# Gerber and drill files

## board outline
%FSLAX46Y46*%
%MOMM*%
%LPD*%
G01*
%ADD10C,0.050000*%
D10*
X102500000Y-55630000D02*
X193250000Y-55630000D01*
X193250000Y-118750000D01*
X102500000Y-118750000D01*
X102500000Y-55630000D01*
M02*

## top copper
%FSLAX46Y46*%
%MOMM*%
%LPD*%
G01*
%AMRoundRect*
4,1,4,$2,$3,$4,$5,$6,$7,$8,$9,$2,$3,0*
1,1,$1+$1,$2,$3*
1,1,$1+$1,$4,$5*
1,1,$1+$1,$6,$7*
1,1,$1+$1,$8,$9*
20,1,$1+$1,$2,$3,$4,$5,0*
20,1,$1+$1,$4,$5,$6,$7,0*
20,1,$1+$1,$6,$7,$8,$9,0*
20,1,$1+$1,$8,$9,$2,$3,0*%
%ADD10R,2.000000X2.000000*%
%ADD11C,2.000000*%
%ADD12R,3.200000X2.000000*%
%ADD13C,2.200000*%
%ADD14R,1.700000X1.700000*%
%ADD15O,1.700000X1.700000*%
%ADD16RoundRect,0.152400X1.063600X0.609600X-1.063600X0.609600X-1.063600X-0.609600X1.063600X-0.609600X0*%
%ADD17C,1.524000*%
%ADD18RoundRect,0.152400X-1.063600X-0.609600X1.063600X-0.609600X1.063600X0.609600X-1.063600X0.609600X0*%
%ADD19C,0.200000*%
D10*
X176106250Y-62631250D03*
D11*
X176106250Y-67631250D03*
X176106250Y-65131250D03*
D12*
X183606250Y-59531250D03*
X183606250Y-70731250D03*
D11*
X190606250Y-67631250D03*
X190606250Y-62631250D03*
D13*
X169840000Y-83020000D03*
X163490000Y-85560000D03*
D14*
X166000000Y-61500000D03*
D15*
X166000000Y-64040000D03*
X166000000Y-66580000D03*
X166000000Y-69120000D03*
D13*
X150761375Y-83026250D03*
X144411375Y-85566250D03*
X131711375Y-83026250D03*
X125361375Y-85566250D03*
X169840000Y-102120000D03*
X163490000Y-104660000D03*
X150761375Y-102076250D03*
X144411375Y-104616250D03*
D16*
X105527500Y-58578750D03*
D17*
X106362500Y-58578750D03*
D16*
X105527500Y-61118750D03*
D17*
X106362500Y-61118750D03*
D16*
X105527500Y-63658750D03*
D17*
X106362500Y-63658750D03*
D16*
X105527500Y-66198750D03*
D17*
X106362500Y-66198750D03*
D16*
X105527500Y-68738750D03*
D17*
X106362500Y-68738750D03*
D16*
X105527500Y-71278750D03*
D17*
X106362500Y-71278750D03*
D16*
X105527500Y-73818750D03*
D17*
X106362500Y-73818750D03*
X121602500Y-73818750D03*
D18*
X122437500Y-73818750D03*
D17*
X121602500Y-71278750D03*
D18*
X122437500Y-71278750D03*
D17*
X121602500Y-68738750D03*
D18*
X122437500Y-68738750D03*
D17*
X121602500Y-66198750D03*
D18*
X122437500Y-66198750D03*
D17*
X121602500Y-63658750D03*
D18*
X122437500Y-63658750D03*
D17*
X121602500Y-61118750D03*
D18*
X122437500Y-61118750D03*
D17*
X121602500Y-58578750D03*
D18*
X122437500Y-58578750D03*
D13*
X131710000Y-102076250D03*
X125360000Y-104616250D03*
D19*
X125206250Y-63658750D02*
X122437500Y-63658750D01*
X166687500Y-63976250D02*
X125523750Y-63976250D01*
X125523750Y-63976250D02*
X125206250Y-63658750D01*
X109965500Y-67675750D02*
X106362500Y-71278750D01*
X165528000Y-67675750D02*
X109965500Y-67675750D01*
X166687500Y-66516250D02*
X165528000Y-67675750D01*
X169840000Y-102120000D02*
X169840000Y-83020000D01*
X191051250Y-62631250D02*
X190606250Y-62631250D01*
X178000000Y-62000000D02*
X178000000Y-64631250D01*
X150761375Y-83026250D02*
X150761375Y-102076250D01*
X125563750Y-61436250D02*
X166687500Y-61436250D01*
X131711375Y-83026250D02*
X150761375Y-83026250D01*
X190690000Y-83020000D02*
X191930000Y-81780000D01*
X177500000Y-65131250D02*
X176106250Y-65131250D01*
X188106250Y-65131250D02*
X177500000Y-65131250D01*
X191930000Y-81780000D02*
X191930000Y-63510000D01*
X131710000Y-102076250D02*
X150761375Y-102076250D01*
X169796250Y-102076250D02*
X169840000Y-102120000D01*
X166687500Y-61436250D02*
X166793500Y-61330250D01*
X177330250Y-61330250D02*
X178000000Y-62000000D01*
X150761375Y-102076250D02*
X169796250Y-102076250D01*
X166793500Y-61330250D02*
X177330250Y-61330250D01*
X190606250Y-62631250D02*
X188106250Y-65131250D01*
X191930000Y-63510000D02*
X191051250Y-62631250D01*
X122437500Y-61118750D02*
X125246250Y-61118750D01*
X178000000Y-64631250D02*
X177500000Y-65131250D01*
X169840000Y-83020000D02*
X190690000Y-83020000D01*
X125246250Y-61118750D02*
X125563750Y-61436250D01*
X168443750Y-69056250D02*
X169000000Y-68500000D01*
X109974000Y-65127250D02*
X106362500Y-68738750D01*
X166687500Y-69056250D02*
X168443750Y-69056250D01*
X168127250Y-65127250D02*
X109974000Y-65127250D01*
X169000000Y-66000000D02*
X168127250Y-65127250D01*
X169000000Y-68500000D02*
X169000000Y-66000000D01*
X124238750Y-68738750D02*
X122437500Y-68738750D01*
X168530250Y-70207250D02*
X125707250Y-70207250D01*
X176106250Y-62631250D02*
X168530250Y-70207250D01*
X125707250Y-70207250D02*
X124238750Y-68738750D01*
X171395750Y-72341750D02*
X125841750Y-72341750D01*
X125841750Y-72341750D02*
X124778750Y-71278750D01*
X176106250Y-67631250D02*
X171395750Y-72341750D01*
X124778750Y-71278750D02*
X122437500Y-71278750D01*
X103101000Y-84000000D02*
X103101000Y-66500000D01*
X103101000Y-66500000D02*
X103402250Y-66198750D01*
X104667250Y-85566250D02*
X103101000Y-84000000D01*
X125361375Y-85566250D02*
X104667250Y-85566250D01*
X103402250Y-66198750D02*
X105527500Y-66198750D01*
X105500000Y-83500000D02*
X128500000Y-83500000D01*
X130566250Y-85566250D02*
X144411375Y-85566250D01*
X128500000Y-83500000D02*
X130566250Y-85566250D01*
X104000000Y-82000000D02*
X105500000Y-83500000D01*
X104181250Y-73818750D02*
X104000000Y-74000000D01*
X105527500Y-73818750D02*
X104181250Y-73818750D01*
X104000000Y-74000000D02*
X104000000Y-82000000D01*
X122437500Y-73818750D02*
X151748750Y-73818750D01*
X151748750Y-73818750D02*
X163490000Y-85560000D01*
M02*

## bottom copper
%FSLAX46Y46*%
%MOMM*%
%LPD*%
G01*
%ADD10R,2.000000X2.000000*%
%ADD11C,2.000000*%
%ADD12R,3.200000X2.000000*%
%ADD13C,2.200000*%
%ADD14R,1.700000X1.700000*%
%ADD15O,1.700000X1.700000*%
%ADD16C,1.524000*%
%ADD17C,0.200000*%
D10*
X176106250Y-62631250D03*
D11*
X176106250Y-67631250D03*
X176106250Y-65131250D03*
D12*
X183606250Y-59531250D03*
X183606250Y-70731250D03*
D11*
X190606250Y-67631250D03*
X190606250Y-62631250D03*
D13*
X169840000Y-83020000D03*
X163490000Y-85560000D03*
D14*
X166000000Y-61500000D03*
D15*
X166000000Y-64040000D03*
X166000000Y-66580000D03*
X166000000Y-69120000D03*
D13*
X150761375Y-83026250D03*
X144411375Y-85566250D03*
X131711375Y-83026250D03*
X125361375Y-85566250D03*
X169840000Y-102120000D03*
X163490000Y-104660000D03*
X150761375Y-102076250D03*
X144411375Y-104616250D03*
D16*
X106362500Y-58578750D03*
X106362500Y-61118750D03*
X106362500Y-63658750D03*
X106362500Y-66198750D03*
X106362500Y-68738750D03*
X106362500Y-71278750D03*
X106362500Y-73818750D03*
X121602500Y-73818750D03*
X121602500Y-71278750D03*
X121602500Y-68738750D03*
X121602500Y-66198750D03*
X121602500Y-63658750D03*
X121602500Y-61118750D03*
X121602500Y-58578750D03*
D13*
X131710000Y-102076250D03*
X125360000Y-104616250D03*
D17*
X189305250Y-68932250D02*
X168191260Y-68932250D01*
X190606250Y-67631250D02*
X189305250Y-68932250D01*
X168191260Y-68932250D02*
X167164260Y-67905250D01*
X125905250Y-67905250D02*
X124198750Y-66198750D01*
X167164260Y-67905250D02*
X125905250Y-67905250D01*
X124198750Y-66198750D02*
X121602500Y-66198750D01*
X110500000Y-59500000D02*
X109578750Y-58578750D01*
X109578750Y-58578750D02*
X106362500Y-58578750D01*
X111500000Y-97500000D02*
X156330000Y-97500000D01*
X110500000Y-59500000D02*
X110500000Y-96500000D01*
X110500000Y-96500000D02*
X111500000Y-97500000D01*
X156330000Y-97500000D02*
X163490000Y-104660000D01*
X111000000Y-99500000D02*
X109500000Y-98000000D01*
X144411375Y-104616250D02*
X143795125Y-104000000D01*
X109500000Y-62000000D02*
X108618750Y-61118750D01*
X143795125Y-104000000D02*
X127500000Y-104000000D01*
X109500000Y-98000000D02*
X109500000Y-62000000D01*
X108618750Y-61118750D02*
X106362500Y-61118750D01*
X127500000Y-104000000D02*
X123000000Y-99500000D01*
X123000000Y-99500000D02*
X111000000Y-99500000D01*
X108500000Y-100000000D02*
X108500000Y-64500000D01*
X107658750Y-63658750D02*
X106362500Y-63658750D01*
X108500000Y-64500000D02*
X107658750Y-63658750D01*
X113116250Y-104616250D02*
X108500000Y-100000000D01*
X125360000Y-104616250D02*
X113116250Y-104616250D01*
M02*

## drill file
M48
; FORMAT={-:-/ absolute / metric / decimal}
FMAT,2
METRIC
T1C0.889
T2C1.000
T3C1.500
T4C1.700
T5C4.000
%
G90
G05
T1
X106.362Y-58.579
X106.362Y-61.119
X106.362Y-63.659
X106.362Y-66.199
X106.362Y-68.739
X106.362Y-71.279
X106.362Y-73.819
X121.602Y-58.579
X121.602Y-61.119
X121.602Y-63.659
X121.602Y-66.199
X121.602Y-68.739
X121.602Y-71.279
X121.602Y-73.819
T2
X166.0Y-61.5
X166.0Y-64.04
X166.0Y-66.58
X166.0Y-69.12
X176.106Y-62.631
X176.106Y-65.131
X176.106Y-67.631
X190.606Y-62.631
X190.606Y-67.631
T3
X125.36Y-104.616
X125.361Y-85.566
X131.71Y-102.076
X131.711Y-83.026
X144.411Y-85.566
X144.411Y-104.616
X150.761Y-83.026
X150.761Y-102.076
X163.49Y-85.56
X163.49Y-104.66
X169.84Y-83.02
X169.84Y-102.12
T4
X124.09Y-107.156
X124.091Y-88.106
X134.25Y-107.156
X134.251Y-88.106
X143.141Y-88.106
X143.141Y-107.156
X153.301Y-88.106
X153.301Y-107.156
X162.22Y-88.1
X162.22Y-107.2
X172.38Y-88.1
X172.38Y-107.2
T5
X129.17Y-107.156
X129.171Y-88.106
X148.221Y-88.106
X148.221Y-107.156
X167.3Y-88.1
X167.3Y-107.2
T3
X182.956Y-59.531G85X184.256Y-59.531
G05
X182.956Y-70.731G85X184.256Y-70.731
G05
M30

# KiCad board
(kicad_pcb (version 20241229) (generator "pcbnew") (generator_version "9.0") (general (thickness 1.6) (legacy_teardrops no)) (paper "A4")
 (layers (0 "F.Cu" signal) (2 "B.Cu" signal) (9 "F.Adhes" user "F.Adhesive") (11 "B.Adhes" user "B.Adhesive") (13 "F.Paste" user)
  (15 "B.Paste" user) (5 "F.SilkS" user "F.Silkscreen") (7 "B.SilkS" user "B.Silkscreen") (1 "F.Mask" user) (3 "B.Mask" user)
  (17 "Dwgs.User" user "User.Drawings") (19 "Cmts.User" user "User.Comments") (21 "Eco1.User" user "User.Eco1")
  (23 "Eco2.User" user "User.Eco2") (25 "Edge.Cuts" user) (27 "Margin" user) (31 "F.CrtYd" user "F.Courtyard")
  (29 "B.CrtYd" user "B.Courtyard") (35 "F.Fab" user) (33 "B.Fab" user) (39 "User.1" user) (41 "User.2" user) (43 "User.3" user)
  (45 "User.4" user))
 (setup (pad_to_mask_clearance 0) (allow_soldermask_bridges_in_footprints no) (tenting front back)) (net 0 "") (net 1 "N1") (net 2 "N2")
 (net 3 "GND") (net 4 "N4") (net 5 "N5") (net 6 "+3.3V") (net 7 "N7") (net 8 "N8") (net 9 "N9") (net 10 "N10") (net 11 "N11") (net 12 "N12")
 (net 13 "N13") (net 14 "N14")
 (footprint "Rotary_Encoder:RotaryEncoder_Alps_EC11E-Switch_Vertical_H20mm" (layer "F.Cu") (at 176.10625 62.63125)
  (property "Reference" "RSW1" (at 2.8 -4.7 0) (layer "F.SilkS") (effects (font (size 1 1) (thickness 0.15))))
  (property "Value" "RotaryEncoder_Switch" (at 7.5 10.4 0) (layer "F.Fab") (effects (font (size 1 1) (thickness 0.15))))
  (pad "A" thru_hole rect (at 0 0) (size 2 2) (drill 1) (layers "*.Cu" "*.Mask") (remove_unused_layers no) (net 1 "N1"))
  (pad "B" thru_hole circle (at 0 5) (size 2 2) (drill 1) (layers "*.Cu" "*.Mask") (remove_unused_layers no) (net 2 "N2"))
  (pad "C" thru_hole circle (at 0 2.5) (size 2 2) (drill 1) (layers "*.Cu" "*.Mask") (remove_unused_layers no) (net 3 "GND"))
  (pad "MP" thru_hole rect (at 7.5 -3.1) (size 3.2 2) (drill oval 2.8 1.5) (layers "*.Cu" "*.Mask") (remove_unused_layers no))
  (pad "MP" thru_hole rect (at 7.5 8.1) (size 3.2 2) (drill oval 2.8 1.5) (layers "*.Cu" "*.Mask") (remove_unused_layers no))
  (pad "S1" thru_hole circle (at 14.5 5) (size 2 2) (drill 1) (layers "*.Cu" "*.Mask") (remove_unused_layers no) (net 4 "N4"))
  (pad "S2" thru_hole circle (at 14.5 0) (size 2 2) (drill 1) (layers "*.Cu" "*.Mask") (remove_unused_layers no) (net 3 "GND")))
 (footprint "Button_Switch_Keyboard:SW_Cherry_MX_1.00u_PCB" (layer "F.Cu") (at 169.84 83.02)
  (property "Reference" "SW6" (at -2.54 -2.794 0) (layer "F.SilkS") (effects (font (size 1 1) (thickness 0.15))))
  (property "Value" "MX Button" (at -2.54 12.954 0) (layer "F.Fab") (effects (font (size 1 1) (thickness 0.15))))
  (pad "" np_thru_hole circle (at -7.62 5.08) (size 1.7 1.7) (drill 1.7) (layers "*.Cu" "*.Mask"))
  (pad "" np_thru_hole circle (at -2.54 5.08) (size 4 4) (drill 4) (layers "*.Cu" "*.Mask"))
  (pad "" np_thru_hole circle (at 2.54 5.08) (size 1.7 1.7) (drill 1.7) (layers "*.Cu" "*.Mask"))
  (pad "1" thru_hole circle (at 0 0) (size 2.2 2.2) (drill 1.5) (layers "*.Cu" "*.Mask") (remove_unused_layers no) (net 3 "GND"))
  (pad "2" thru_hole circle (at -6.35 2.54) (size 2.2 2.2) (drill 1.5) (layers "*.Cu" "*.Mask") (remove_unused_layers no) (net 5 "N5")))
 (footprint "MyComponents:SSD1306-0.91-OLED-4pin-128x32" (layer "F.Cu") (at 129.5 59.31)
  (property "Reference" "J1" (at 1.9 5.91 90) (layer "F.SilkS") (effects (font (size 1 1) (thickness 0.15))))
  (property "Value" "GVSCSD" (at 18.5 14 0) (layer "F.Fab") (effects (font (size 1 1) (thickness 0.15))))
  (pad "1" thru_hole rect (at 36.5 2.19) (size 1.7 1.7) (drill 1) (layers "*.Cu" "*.Mask") (remove_unused_layers no) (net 3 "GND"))
  (pad "2" thru_hole oval (at 36.5 4.73) (size 1.7 1.7) (drill 1) (layers "*.Cu" "*.Mask") (remove_unused_layers no) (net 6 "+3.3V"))
  (pad "3" thru_hole oval (at 36.5 7.27) (size 1.7 1.7) (drill 1) (layers "*.Cu" "*.Mask") (remove_unused_layers no) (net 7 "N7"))
  (pad "4" thru_hole oval (at 36.5 9.81) (size 1.7 1.7) (drill 1) (layers "*.Cu" "*.Mask") (remove_unused_layers no) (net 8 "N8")))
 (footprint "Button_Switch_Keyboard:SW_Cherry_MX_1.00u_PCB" (layer "F.Cu") (at 150.761375 83.02625)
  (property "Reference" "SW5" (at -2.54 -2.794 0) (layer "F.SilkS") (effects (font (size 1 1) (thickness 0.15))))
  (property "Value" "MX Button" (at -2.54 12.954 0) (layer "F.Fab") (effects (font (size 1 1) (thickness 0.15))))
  (pad "" np_thru_hole circle (at -7.62 5.08) (size 1.7 1.7) (drill 1.7) (layers "*.Cu" "*.Mask"))
  (pad "" np_thru_hole circle (at -2.54 5.08) (size 4 4) (drill 4) (layers "*.Cu" "*.Mask"))
  (pad "" np_thru_hole circle (at 2.54 5.08) (size 1.7 1.7) (drill 1.7) (layers "*.Cu" "*.Mask"))
  (pad "1" thru_hole circle (at 0 0) (size 2.2 2.2) (drill 1.5) (layers "*.Cu" "*.Mask") (remove_unused_layers no) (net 3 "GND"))
  (pad "2" thru_hole circle (at -6.35 2.54) (size 2.2 2.2) (drill 1.5) (layers "*.Cu" "*.Mask") (remove_unused_layers no) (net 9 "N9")))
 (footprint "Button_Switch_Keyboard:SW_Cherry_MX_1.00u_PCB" (layer "F.Cu") (at 131.711375 83.02625)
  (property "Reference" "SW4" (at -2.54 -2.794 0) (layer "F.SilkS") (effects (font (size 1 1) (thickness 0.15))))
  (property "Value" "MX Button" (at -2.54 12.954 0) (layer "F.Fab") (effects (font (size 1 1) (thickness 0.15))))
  (pad "" np_thru_hole circle (at -7.62 5.08) (size 1.7 1.7) (drill 1.7) (layers "*.Cu" "*.Mask"))
  (pad "" np_thru_hole circle (at -2.54 5.08) (size 4 4) (drill 4) (layers "*.Cu" "*.Mask"))
  (pad "" np_thru_hole circle (at 2.54 5.08) (size 1.7 1.7) (drill 1.7) (layers "*.Cu" "*.Mask"))
  (pad "1" thru_hole circle (at 0 0) (size 2.2 2.2) (drill 1.5) (layers "*.Cu" "*.Mask") (remove_unused_layers no) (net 3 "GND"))
  (pad "2" thru_hole circle (at -6.35 2.54) (size 2.2 2.2) (drill 1.5) (layers "*.Cu" "*.Mask") (remove_unused_layers no) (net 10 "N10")))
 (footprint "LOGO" (layer "F.Cu") (at 186.96 112.6)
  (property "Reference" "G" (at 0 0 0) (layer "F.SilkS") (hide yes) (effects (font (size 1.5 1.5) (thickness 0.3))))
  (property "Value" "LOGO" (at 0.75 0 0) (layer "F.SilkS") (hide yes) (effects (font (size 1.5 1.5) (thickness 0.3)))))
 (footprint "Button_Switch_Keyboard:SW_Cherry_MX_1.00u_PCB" (layer "F.Cu") (at 169.84 102.12)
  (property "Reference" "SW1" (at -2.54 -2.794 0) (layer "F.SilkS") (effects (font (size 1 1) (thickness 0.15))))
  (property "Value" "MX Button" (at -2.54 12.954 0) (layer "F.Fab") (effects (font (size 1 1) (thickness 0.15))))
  (pad "" np_thru_hole circle (at -7.62 5.08) (size 1.7 1.7) (drill 1.7) (layers "*.Cu" "*.Mask"))
  (pad "" np_thru_hole circle (at -2.54 5.08) (size 4 4) (drill 4) (layers "*.Cu" "*.Mask"))
  (pad "" np_thru_hole circle (at 2.54 5.08) (size 1.7 1.7) (drill 1.7) (layers "*.Cu" "*.Mask"))
  (pad "1" thru_hole circle (at 0 0) (size 2.2 2.2) (drill 1.5) (layers "*.Cu" "*.Mask") (remove_unused_layers no) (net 3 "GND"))
  (pad "2" thru_hole circle (at -6.35 2.54) (size 2.2 2.2) (drill 1.5) (layers "*.Cu" "*.Mask") (remove_unused_layers no) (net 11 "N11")))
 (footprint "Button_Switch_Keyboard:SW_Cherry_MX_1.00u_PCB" (layer "F.Cu") (at 150.761375 102.07625)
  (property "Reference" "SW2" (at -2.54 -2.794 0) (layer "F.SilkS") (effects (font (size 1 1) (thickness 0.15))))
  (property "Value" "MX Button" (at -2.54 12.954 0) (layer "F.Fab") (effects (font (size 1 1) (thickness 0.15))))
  (pad "" np_thru_hole circle (at -7.62 5.08) (size 1.7 1.7) (drill 1.7) (layers "*.Cu" "*.Mask"))
  (pad "" np_thru_hole circle (at -2.54 5.08) (size 4 4) (drill 4) (layers "*.Cu" "*.Mask"))
  (pad "" np_thru_hole circle (at 2.54 5.08) (size 1.7 1.7) (drill 1.7) (layers "*.Cu" "*.Mask"))
  (pad "1" thru_hole circle (at 0 0) (size 2.2 2.2) (drill 1.5) (layers "*.Cu" "*.Mask") (remove_unused_layers no) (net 3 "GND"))
  (pad "2" thru_hole circle (at -6.35 2.54) (size 2.2 2.2) (drill 1.5) (layers "*.Cu" "*.Mask") (remove_unused_layers no) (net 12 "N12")))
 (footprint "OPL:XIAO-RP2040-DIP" (layer "F.Cu") (at 113.9825 66.19875)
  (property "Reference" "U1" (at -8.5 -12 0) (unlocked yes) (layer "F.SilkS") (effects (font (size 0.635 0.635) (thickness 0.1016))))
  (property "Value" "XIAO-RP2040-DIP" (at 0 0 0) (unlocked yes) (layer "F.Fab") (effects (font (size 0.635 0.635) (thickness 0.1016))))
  (pad "1" smd roundrect (at -8.455 -7.62 180) (size 2.432 1.524) (layers "F.Cu" "F.Mask") (roundrect_rratio 0.1) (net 11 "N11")
   (thermal_bridge_angle 45))
  (pad "1" thru_hole circle (at -7.62 -7.62 180) (size 1.524 1.524) (drill 0.889) (layers "*.Cu" "*.Mask") (remove_unused_layers no)
   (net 11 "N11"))
  (pad "2" smd roundrect (at -8.455 -5.08 180) (size 2.432 1.524) (layers "F.Cu" "F.Mask") (roundrect_rratio 0.1) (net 12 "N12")
   (thermal_bridge_angle 45))
  (pad "2" thru_hole circle (at -7.62 -5.08 180) (size 1.524 1.524) (drill 0.889) (layers "*.Cu" "*.Mask") (remove_unused_layers no)
   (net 12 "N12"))
  (pad "3" smd roundrect (at -8.455 -2.54 180) (size 2.432 1.524) (layers "F.Cu" "F.Mask") (roundrect_rratio 0.1) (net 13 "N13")
   (thermal_bridge_angle 45))
  (pad "3" thru_hole circle (at -7.62 -2.54 180) (size 1.524 1.524) (drill 0.889) (layers "*.Cu" "*.Mask") (remove_unused_layers no)
   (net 13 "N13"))
  (pad "4" smd roundrect (at -8.455 0 180) (size 2.432 1.524) (layers "F.Cu" "F.Mask") (roundrect_rratio 0.1) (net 10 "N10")
   (thermal_bridge_angle 45))
  (pad "4" thru_hole circle (at -7.62 0 180) (size 1.524 1.524) (drill 0.889) (layers "*.Cu" "*.Mask") (remove_unused_layers no)
   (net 10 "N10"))
  (pad "5" smd roundrect (at -8.455 2.54 180) (size 2.432 1.524) (layers "F.Cu" "F.Mask") (roundrect_rratio 0.1) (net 8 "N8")
   (thermal_bridge_angle 45))
  (pad "5" thru_hole circle (at -7.62 2.54 180) (size 1.524 1.524) (drill 0.889) (layers "*.Cu" "*.Mask") (remove_unused_layers no)
   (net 8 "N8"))
  (pad "6" smd roundrect (at -8.455 5.08 180) (size 2.432 1.524) (layers "F.Cu" "F.Mask") (roundrect_rratio 0.1) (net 7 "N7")
   (thermal_bridge_angle 45))
  (pad "6" thru_hole circle (at -7.62 5.08 180) (size 1.524 1.524) (drill 0.889) (layers "*.Cu" "*.Mask") (remove_unused_layers no)
   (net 7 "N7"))
  (pad "7" smd roundrect (at -8.455 7.62 180) (size 2.432 1.524) (layers "F.Cu" "F.Mask") (roundrect_rratio 0.1) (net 9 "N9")
   (thermal_bridge_angle 45))
  (pad "7" thru_hole circle (at -7.62 7.62 180) (size 1.524 1.524) (drill 0.889) (layers "*.Cu" "*.Mask") (remove_unused_layers no)
   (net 9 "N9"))
  (pad "8" thru_hole circle (at 7.62 7.62) (size 1.524 1.524) (drill 0.889) (layers "*.Cu" "*.Mask") (remove_unused_layers no) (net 5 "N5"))
  (pad "8" smd roundrect (at 8.455 7.62) (size 2.432 1.524) (layers "F.Cu" "F.Mask") (roundrect_rratio 0.1) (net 5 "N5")
   (thermal_bridge_angle 45))
  (pad "9" thru_hole circle (at 7.62 5.08) (size 1.524 1.524) (drill 0.889) (layers "*.Cu" "*.Mask") (remove_unused_layers no) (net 2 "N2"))
  (pad "9" smd roundrect (at 8.455 5.08) (size 2.432 1.524) (layers "F.Cu" "F.Mask") (roundrect_rratio 0.1) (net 2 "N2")
   (thermal_bridge_angle 45))
  (pad "10" thru_hole circle (at 7.62 2.54) (size 1.524 1.524) (drill 0.889) (layers "*.Cu" "*.Mask") (remove_unused_layers no) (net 1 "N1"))
  (pad "10" smd roundrect (at 8.455 2.54) (size 2.432 1.524) (layers "F.Cu" "F.Mask") (roundrect_rratio 0.1) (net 1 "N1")
   (thermal_bridge_angle 45))
  (pad "11" thru_hole circle (at 7.62 0) (size 1.524 1.524) (drill 0.889) (layers "*.Cu" "*.Mask") (remove_unused_layers no) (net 4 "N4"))
  (pad "11" smd roundrect (at 8.455 0) (size 2.432 1.524) (layers "F.Cu" "F.Mask") (roundrect_rratio 0.1) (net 4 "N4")
   (thermal_bridge_angle 45))
  (pad "12" thru_hole circle (at 7.62 -2.54) (size 1.524 1.524) (drill 0.889) (layers "*.Cu" "*.Mask") (remove_unused_layers no)
   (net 6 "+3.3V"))
  (pad "12" smd roundrect (at 8.455 -2.54) (size 2.432 1.524) (layers "F.Cu" "F.Mask") (roundrect_rratio 0.1) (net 6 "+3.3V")
   (thermal_bridge_angle 45))
  (pad "13" thru_hole circle (at 7.62 -5.08) (size 1.524 1.524) (drill 0.889) (layers "*.Cu" "*.Mask") (remove_unused_layers no)
   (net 3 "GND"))
  (pad "13" smd roundrect (at 8.455 -5.08) (size 2.432 1.524) (layers "F.Cu" "F.Mask") (roundrect_rratio 0.1) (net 3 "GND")
   (thermal_bridge_angle 45))
  (pad "14" thru_hole circle (at 7.62 -7.62) (size 1.524 1.524) (drill 0.889) (layers "*.Cu" "*.Mask") (remove_unused_layers no)
   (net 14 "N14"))
  (pad "14" smd roundrect (at 8.455 -7.62) (size 2.432 1.524) (layers "F.Cu" "F.Mask") (roundrect_rratio 0.1) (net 14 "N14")
   (thermal_bridge_angle 45)))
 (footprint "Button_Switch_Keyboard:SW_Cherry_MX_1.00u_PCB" (layer "F.Cu") (at 131.71 102.07625)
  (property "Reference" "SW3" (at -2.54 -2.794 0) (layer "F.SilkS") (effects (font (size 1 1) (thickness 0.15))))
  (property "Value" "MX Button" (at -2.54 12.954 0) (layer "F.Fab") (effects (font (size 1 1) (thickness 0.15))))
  (pad "" np_thru_hole circle (at -7.62 5.08) (size 1.7 1.7) (drill 1.7) (layers "*.Cu" "*.Mask"))
  (pad "" np_thru_hole circle (at -2.54 5.08) (size 4 4) (drill 4) (layers "*.Cu" "*.Mask"))
  (pad "" np_thru_hole circle (at 2.54 5.08) (size 1.7 1.7) (drill 1.7) (layers "*.Cu" "*.Mask"))
  (pad "1" thru_hole circle (at 0 0) (size 2.2 2.2) (drill 1.5) (layers "*.Cu" "*.Mask") (remove_unused_layers no) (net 3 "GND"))
  (pad "2" thru_hole circle (at -6.35 2.54) (size 2.2 2.2) (drill 1.5) (layers "*.Cu" "*.Mask") (remove_unused_layers no) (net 13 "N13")))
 (gr_rect (start 102.5 55.63) (end 193.25 118.75) (stroke (width 0.05) (type default)) (fill no) (layer "Edge.Cuts"))
 (segment (start 125.20625 63.65875) (end 122.4375 63.65875) (width 0.2) (layer "F.Cu") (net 6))
 (segment (start 166.6875 63.97625) (end 125.52375 63.97625) (width 0.2) (layer "F.Cu") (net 6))
 (segment (start 125.52375 63.97625) (end 125.20625 63.65875) (width 0.2) (layer "F.Cu") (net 6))
 (segment (start 109.9655 67.67575) (end 106.3625 71.27875) (width 0.2) (layer "F.Cu") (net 7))
 (segment (start 165.528 67.67575) (end 109.9655 67.67575) (width 0.2) (layer "F.Cu") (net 7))
 (segment (start 166.6875 66.51625) (end 165.528 67.67575) (width 0.2) (layer "F.Cu") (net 7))
 (segment (start 169.84 102.12) (end 169.84 83.02) (width 0.2) (layer "F.Cu") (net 3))
 (segment (start 191.05125 62.63125) (end 190.60625 62.63125) (width 0.2) (layer "F.Cu") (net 3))
 (segment (start 178 62) (end 178 64.63125) (width 0.2) (layer "F.Cu") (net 3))
 (segment (start 150.761375 83.02625) (end 150.761375 102.07625) (width 0.2) (layer "F.Cu") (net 3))
 (segment (start 125.56375 61.43625) (end 166.6875 61.43625) (width 0.2) (layer "F.Cu") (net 3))
 (segment (start 131.711375 83.02625) (end 150.761375 83.02625) (width 0.2) (layer "F.Cu") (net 3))
 (segment (start 190.69 83.02) (end 191.93 81.78) (width 0.2) (layer "F.Cu") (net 3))
 (segment (start 177.5 65.13125) (end 176.10625 65.13125) (width 0.2) (layer "F.Cu") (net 3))
 (segment (start 188.10625 65.13125) (end 177.5 65.13125) (width 0.2) (layer "F.Cu") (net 3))
 (segment (start 191.93 81.78) (end 191.93 63.51) (width 0.2) (layer "F.Cu") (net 3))
 (segment (start 131.71 102.07625) (end 150.761375 102.07625) (width 0.2) (layer "F.Cu") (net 3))
 (segment (start 169.79625 102.07625) (end 169.84 102.12) (width 0.2) (layer "F.Cu") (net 3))
 (segment (start 166.6875 61.43625) (end 166.7935 61.33025) (width 0.2) (layer "F.Cu") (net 3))
 (segment (start 177.33025 61.33025) (end 178 62) (width 0.2) (layer "F.Cu") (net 3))
 (segment (start 150.761375 102.07625) (end 169.79625 102.07625) (width 0.2) (layer "F.Cu") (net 3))
 (segment (start 166.7935 61.33025) (end 177.33025 61.33025) (width 0.2) (layer "F.Cu") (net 3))
 (segment (start 190.60625 62.63125) (end 188.10625 65.13125) (width 0.2) (layer "F.Cu") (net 3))
 (segment (start 191.93 63.51) (end 191.05125 62.63125) (width 0.2) (layer "F.Cu") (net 3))
 (segment (start 122.4375 61.11875) (end 125.24625 61.11875) (width 0.2) (layer "F.Cu") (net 3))
 (segment (start 178 64.63125) (end 177.5 65.13125) (width 0.2) (layer "F.Cu") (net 3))
 (segment (start 169.84 83.02) (end 190.69 83.02) (width 0.2) (layer "F.Cu") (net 3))
 (segment (start 125.24625 61.11875) (end 125.56375 61.43625) (width 0.2) (layer "F.Cu") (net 3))
 (segment (start 168.44375 69.05625) (end 169 68.5) (width 0.2) (layer "F.Cu") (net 8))
 (segment (start 109.974 65.12725) (end 106.3625 68.73875) (width 0.2) (layer "F.Cu") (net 8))
 (segment (start 166.6875 69.05625) (end 168.44375 69.05625) (width 0.2) (layer "F.Cu") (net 8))
 (segment (start 168.12725 65.12725) (end 109.974 65.12725) (width 0.2) (layer "F.Cu") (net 8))
 (segment (start 169 66) (end 168.12725 65.12725) (width 0.2) (layer "F.Cu") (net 8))
 (segment (start 169 68.5) (end 169 66) (width 0.2) (layer "F.Cu") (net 8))
 (segment (start 189.30525 68.93225) (end 168.19126 68.93225) (width 0.2) (layer "B.Cu") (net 4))
 (segment (start 190.60625 67.63125) (end 189.30525 68.93225) (width 0.2) (layer "B.Cu") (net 4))
 (segment (start 168.19126 68.93225) (end 167.16426 67.90525) (width 0.2) (layer "B.Cu") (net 4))
 (segment (start 125.90525 67.90525) (end 124.19875 66.19875) (width 0.2) (layer "B.Cu") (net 4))
 (segment (start 167.16426 67.90525) (end 125.90525 67.90525) (width 0.2) (layer "B.Cu") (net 4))
 (segment (start 124.19875 66.19875) (end 121.6025 66.19875) (width 0.2) (layer "B.Cu") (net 4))
 (segment (start 124.23875 68.73875) (end 122.4375 68.73875) (width 0.2) (layer "F.Cu") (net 1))
 (segment (start 168.53025 70.20725) (end 125.70725 70.20725) (width 0.2) (layer "F.Cu") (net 1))
 (segment (start 176.10625 62.63125) (end 168.53025 70.20725) (width 0.2) (layer "F.Cu") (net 1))
 (segment (start 125.70725 70.20725) (end 124.23875 68.73875) (width 0.2) (layer "F.Cu") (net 1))
 (segment (start 171.39575 72.34175) (end 125.84175 72.34175) (width 0.2) (layer "F.Cu") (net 2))
 (segment (start 125.84175 72.34175) (end 124.77875 71.27875) (width 0.2) (layer "F.Cu") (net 2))
 (segment (start 176.10625 67.63125) (end 171.39575 72.34175) (width 0.2) (layer "F.Cu") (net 2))
 (segment (start 124.77875 71.27875) (end 122.4375 71.27875) (width 0.2) (layer "F.Cu") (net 2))
 (segment (start 110.5 59.5) (end 109.57875 58.57875) (width 0.2) (layer "B.Cu") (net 11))
 (segment (start 109.57875 58.57875) (end 106.3625 58.57875) (width 0.2) (layer "B.Cu") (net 11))
 (segment (start 111.5 97.5) (end 156.33 97.5) (width 0.2) (layer "B.Cu") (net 11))
 (segment (start 110.5 59.5) (end 110.5 96.5) (width 0.2) (layer "B.Cu") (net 11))
 (segment (start 110.5 96.5) (end 111.5 97.5) (width 0.2) (layer "B.Cu") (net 11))
 (segment (start 156.33 97.5) (end 163.49 104.66) (width 0.2) (layer "B.Cu") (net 11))
 (segment (start 111 99.5) (end 109.5 98) (width 0.2) (layer "B.Cu") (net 12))
 (segment (start 144.411375 104.61625) (end 143.795125 104) (width 0.2) (layer "B.Cu") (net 12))
 (segment (start 109.5 62) (end 108.61875 61.11875) (width 0.2) (layer "B.Cu") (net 12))
 (segment (start 143.795125 104) (end 127.5 104) (width 0.2) (layer "B.Cu") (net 12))
 (segment (start 109.5 98) (end 109.5 62) (width 0.2) (layer "B.Cu") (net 12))
 (segment (start 108.61875 61.11875) (end 106.3625 61.11875) (width 0.2) (layer "B.Cu") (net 12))
 (segment (start 127.5 104) (end 123 99.5) (width 0.2) (layer "B.Cu") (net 12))
 (segment (start 123 99.5) (end 111 99.5) (width 0.2) (layer "B.Cu") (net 12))
 (segment (start 108.5 100) (end 108.5 64.5) (width 0.2) (layer "B.Cu") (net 13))
 (segment (start 107.65875 63.65875) (end 106.3625 63.65875) (width 0.2) (layer "B.Cu") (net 13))
 (segment (start 108.5 64.5) (end 107.65875 63.65875) (width 0.2) (layer "B.Cu") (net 13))
 (segment (start 113.11625 104.61625) (end 108.5 100) (width 0.2) (layer "B.Cu") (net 13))
 (segment (start 125.36 104.61625) (end 113.11625 104.61625) (width 0.2) (layer "B.Cu") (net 13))
 (segment (start 103.101 84) (end 103.101 66.5) (width 0.2) (layer "F.Cu") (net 10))
 (segment (start 103.101 66.5) (end 103.40225 66.19875) (width 0.2) (layer "F.Cu") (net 10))
 (segment (start 104.66725 85.56625) (end 103.101 84) (width 0.2) (layer "F.Cu") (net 10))
 (segment (start 125.361375 85.56625) (end 104.66725 85.56625) (width 0.2) (layer "F.Cu") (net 10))
 (segment (start 103.40225 66.19875) (end 105.5275 66.19875) (width 0.2) (layer "F.Cu") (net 10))
 (segment (start 105.5 83.5) (end 128.5 83.5) (width 0.2) (layer "F.Cu") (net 9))
 (segment (start 130.56625 85.56625) (end 144.411375 85.56625) (width 0.2) (layer "F.Cu") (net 9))
 (segment (start 128.5 83.5) (end 130.56625 85.56625) (width 0.2) (layer "F.Cu") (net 9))
 (segment (start 104 82) (end 105.5 83.5) (width 0.2) (layer "F.Cu") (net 9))
 (segment (start 104.18125 73.81875) (end 104 74) (width 0.2) (layer "F.Cu") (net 9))
 (segment (start 105.5275 73.81875) (end 104.18125 73.81875) (width 0.2) (layer "F.Cu") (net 9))
 (segment (start 104 74) (end 104 82) (width 0.2) (layer "F.Cu") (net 9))
 (segment (start 122.4375 73.81875) (end 151.74875 73.81875) (width 0.2) (layer "F.Cu") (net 5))
 (segment (start 151.74875 73.81875) (end 163.49 85.56) (width 0.2) (layer "F.Cu") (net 5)))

